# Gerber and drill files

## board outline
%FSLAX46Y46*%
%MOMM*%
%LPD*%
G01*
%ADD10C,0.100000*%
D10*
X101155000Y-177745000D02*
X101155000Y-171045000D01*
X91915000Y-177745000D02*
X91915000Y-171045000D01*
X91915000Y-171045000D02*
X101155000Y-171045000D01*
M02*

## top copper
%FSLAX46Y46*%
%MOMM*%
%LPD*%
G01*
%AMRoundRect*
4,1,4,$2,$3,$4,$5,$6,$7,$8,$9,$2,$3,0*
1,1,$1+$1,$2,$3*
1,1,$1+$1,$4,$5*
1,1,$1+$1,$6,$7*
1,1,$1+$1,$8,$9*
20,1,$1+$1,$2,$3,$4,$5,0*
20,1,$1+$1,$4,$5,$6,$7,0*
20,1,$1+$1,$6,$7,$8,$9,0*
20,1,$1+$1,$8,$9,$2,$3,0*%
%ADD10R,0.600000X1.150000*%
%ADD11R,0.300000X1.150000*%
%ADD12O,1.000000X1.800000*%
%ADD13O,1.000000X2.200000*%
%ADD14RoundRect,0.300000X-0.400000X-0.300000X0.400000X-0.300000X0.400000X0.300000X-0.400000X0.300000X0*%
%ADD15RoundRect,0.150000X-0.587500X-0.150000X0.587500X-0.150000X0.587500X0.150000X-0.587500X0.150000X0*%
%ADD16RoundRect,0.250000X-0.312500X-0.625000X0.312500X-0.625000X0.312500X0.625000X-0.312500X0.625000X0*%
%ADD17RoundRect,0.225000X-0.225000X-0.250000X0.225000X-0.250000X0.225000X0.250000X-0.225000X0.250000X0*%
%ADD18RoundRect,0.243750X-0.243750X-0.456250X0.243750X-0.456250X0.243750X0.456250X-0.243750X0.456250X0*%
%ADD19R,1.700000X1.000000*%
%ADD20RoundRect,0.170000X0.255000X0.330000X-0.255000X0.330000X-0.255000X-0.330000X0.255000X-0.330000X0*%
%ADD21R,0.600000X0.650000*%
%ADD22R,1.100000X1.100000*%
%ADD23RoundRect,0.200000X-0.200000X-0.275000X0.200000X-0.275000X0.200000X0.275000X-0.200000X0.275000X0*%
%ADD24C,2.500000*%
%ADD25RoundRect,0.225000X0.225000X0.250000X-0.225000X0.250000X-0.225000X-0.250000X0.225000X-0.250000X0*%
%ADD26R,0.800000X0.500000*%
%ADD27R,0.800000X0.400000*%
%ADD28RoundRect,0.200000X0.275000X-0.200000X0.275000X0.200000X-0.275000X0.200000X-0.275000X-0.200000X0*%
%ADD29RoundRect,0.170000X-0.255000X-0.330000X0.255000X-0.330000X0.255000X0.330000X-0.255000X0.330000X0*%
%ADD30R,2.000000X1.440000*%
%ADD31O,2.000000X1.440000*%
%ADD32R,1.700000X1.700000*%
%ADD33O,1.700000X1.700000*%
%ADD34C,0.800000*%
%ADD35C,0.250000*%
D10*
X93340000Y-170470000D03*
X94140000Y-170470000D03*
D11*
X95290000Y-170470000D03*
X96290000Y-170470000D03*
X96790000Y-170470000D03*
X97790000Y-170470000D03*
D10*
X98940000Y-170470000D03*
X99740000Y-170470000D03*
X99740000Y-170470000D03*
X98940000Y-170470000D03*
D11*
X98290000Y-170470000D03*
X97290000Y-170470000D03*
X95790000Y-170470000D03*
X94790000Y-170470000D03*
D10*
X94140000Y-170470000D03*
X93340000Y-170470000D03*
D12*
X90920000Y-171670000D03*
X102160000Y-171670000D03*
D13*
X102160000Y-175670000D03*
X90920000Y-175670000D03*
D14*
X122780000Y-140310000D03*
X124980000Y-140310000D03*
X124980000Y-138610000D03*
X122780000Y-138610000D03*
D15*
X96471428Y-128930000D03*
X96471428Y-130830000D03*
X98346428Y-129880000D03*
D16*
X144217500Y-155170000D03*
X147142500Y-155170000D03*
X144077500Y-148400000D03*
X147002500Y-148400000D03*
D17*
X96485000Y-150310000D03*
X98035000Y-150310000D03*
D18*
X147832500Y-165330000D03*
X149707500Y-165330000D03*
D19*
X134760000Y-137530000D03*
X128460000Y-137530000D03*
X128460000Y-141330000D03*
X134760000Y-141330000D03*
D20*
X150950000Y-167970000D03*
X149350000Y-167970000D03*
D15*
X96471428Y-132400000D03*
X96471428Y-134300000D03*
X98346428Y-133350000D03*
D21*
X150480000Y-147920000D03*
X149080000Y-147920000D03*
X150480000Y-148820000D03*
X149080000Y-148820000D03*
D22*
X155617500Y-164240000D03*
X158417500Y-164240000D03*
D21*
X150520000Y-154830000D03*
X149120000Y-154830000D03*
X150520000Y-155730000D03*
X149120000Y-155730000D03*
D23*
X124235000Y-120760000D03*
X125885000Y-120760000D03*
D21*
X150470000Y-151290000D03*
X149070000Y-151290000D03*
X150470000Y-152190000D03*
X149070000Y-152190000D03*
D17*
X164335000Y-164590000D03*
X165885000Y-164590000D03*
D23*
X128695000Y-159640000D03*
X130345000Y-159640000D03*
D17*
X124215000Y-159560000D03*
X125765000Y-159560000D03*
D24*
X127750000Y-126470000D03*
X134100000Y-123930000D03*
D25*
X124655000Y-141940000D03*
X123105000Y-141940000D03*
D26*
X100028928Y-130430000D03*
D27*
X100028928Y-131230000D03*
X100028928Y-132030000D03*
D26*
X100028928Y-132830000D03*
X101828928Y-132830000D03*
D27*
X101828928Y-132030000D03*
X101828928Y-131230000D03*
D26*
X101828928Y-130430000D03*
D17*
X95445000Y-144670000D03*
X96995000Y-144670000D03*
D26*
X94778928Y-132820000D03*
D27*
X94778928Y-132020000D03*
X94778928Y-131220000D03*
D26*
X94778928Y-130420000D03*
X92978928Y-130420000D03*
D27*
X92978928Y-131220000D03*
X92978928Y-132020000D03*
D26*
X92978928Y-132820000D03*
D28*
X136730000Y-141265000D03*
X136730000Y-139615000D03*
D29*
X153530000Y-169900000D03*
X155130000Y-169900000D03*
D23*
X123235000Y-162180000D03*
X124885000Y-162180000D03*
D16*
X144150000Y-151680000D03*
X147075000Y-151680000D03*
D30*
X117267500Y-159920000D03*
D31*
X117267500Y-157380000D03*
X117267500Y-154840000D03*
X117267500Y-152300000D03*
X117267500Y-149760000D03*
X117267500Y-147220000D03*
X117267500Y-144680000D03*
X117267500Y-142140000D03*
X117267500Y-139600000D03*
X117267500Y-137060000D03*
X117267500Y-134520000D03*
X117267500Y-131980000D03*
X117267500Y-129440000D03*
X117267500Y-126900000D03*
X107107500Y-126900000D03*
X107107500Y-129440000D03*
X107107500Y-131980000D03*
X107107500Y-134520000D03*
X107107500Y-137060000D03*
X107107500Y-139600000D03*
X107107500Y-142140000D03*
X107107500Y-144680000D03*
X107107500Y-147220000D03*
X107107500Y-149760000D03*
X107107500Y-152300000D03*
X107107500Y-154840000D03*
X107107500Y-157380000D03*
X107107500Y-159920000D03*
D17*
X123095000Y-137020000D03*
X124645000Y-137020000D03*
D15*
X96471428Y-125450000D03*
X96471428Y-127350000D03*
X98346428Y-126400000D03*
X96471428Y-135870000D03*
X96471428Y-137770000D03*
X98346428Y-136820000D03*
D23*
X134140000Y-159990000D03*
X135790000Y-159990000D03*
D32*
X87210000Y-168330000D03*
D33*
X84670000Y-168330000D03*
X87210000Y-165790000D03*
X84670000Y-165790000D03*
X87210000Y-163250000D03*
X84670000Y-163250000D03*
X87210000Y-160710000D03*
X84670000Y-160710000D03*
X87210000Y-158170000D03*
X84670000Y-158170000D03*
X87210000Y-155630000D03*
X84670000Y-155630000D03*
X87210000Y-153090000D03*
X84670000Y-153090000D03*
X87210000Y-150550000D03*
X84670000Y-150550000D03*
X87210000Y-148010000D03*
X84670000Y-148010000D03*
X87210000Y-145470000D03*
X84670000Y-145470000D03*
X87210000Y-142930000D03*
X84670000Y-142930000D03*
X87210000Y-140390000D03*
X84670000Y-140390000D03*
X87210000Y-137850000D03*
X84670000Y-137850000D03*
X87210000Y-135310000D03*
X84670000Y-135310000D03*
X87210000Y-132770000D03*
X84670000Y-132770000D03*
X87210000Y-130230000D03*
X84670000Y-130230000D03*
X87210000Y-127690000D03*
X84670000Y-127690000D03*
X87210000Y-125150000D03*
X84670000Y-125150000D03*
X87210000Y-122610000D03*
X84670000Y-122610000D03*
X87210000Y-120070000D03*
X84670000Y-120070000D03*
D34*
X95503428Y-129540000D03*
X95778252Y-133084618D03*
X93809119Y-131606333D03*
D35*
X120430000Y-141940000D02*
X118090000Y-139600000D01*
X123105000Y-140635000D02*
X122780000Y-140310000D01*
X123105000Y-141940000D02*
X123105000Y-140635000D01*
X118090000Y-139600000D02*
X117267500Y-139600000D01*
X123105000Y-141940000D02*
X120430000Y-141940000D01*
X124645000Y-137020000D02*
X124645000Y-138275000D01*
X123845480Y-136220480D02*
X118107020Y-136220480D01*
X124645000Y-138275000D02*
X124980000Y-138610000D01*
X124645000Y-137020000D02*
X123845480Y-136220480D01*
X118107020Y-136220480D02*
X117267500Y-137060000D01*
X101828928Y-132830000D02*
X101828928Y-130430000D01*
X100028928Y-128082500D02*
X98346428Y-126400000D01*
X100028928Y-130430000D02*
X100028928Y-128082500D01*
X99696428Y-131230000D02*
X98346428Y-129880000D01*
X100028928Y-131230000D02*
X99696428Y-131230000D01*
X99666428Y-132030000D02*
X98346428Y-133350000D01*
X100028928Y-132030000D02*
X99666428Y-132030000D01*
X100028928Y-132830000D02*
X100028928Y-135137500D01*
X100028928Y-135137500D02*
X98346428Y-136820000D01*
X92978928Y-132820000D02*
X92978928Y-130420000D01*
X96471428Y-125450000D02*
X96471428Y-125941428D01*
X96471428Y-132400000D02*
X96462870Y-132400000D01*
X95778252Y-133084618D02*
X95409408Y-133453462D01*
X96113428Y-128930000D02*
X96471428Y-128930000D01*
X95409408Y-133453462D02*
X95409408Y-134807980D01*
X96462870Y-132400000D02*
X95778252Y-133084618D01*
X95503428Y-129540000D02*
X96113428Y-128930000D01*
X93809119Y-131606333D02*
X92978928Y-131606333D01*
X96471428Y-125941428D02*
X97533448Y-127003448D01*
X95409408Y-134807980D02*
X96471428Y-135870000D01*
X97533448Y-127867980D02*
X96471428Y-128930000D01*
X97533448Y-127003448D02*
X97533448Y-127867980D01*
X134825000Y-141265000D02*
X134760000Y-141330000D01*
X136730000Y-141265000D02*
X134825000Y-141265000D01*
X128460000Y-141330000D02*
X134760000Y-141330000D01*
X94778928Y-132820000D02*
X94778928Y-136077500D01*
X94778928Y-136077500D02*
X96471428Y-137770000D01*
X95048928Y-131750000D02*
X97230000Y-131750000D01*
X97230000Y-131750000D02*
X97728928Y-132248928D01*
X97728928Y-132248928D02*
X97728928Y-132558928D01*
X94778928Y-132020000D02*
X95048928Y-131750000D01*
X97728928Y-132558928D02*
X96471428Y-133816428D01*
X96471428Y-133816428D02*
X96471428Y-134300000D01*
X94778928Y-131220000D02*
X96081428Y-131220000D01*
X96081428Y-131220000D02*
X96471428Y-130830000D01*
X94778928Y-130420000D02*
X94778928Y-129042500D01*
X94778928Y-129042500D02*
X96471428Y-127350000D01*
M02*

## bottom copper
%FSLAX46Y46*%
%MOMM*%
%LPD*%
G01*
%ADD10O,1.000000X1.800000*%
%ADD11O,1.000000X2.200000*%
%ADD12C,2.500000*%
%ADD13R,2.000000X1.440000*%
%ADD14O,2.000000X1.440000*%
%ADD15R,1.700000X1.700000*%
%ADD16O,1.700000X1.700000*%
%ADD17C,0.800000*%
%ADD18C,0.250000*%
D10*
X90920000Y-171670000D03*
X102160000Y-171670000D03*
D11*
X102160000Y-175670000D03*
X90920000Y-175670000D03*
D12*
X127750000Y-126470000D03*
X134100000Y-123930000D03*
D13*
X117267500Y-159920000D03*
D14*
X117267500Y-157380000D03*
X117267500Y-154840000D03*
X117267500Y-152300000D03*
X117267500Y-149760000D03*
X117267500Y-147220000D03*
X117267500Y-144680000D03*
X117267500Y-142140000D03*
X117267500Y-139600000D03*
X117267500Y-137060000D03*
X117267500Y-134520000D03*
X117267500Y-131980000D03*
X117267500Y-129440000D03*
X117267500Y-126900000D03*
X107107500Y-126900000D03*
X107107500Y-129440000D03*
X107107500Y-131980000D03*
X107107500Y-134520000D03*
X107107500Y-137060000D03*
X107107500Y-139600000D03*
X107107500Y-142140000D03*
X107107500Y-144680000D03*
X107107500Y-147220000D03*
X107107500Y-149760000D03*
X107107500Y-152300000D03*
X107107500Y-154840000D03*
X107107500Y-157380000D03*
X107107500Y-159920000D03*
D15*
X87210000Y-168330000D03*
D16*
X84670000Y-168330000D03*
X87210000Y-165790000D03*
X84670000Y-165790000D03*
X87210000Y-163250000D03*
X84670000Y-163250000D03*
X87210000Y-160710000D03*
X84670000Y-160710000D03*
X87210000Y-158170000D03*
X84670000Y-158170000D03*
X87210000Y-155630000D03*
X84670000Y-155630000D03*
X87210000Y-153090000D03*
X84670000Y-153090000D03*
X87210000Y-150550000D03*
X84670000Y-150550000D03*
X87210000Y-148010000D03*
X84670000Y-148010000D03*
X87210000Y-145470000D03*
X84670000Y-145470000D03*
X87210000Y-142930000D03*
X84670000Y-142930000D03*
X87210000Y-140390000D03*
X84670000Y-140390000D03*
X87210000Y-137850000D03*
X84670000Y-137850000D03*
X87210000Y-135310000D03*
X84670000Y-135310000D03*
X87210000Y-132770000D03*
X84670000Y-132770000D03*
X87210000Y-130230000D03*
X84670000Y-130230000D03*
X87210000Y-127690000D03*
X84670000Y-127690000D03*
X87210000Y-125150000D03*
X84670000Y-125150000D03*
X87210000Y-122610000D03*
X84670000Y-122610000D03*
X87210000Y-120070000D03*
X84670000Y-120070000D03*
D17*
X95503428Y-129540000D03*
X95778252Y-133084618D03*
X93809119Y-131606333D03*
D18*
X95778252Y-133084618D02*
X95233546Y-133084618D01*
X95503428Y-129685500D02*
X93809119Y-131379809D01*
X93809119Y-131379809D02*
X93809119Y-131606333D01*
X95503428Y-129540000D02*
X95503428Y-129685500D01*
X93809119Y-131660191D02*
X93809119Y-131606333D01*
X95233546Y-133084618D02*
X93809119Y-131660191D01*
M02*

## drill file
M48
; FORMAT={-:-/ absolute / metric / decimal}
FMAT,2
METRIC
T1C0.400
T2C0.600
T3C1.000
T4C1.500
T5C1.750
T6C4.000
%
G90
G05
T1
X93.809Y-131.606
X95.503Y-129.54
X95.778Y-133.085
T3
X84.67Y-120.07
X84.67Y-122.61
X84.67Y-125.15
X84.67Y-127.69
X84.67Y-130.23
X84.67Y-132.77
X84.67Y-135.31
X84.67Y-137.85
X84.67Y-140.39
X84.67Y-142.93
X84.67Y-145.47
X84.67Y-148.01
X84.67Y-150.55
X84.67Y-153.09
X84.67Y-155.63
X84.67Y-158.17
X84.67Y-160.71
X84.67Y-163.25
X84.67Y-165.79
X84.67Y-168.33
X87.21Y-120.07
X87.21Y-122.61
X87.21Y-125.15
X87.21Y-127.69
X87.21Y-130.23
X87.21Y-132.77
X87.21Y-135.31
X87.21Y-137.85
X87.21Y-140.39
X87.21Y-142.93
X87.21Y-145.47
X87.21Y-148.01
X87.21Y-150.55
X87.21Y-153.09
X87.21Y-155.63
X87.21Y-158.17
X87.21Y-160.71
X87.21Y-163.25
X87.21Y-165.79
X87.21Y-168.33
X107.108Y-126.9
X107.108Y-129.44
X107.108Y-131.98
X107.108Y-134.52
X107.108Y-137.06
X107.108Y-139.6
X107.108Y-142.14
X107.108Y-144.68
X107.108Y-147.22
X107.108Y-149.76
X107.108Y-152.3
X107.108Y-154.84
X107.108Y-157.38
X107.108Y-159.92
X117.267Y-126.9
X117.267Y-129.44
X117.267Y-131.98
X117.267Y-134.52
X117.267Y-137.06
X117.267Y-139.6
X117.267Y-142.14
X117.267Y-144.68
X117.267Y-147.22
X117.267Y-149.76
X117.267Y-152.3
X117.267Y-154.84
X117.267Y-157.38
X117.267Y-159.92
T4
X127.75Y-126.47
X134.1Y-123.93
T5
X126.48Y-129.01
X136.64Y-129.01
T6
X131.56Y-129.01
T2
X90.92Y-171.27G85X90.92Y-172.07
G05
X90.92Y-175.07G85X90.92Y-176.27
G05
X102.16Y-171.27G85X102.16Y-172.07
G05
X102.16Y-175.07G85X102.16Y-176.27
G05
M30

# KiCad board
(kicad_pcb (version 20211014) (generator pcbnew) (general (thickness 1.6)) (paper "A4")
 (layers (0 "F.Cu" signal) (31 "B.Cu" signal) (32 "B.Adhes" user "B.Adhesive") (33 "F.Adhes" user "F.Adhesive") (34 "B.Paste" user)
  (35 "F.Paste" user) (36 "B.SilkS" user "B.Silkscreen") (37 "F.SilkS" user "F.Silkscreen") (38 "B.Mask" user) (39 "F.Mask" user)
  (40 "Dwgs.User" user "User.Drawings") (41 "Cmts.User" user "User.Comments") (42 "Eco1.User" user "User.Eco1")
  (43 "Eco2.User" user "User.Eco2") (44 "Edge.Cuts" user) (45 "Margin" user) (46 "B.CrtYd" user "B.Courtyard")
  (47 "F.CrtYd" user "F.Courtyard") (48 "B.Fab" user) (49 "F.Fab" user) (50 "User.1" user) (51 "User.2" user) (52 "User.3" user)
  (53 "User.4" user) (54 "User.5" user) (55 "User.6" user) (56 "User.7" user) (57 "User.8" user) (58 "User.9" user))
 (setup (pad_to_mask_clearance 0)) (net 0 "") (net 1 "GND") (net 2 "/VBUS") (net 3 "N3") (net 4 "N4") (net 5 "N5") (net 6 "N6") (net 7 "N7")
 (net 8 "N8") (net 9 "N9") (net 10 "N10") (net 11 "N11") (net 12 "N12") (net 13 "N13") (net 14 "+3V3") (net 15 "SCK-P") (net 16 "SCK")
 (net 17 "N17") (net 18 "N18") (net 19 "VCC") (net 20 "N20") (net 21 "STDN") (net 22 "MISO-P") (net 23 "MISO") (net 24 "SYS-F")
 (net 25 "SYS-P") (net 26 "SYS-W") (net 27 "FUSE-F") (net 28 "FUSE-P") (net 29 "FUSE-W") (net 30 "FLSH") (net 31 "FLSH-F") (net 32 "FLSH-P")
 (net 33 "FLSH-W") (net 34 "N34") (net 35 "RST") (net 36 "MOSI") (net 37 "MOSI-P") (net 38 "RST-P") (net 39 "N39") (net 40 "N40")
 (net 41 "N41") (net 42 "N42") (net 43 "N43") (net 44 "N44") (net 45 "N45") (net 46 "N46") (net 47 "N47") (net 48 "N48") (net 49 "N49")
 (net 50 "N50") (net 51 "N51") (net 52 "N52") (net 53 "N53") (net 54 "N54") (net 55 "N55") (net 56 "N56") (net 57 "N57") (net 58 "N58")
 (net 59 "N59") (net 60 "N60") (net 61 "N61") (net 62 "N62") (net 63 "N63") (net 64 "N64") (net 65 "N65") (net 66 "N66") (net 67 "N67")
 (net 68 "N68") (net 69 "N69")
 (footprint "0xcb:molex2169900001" (layer "F.Cu") (at 96.54 177.77)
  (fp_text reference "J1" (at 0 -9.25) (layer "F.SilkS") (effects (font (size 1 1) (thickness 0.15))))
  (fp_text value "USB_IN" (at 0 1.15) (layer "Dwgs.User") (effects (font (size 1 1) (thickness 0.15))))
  (fp_line (start 4.615 -0.025) (end 4.615 -6.725) (layer "Edge.Cuts") (width 0.1))
  (fp_line (start -4.625 -0.025) (end -4.625 -6.725) (layer "Edge.Cuts") (width 0.1))
  (fp_line (start -4.625 -6.725) (end 4.615 -6.725) (layer "Edge.Cuts") (width 0.1))
  (pad "A1" smd rect (at -3.2 -7.3) (size 0.6 1.15) (layers "F.Cu" "F.Paste" "F.Mask") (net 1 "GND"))
  (pad "A4" smd rect (at -2.4 -7.3) (size 0.6 1.15) (layers "F.Cu" "F.Paste" "F.Mask") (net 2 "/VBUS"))
  (pad "A5" smd rect (at -1.25 -7.3) (size 0.3 1.15) (layers "F.Cu" "F.Paste" "F.Mask") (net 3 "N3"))
  (pad "A6" smd rect (at -0.25 -7.3) (size 0.3 1.15) (layers "F.Cu" "F.Paste" "F.Mask") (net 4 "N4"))
  (pad "A7" smd rect (at 0.25 -7.3) (size 0.3 1.15) (layers "F.Cu" "F.Paste" "F.Mask") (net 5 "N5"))
  (pad "A8" smd rect (at 1.25 -7.3) (size 0.3 1.15) (layers "F.Cu" "F.Paste" "F.Mask") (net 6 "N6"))
  (pad "A9" smd rect (at 2.4 -7.3) (size 0.6 1.15) (layers "F.Cu" "F.Paste" "F.Mask") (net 2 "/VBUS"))
  (pad "A12" smd rect (at 3.2 -7.3) (size 0.6 1.15) (layers "F.Cu" "F.Paste" "F.Mask") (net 1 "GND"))
  (pad "B1" smd rect (at 3.2 -7.3) (size 0.6 1.15) (layers "F.Cu" "F.Paste" "F.Mask") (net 1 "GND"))
  (pad "B4" smd rect (at 2.4 -7.3) (size 0.6 1.15) (layers "F.Cu" "F.Paste" "F.Mask") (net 2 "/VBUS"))
  (pad "B5" smd rect (at 1.75 -7.3) (size 0.3 1.15) (layers "F.Cu" "F.Paste" "F.Mask") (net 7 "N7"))
  (pad "B6" smd rect (at 0.75 -7.3) (size 0.3 1.15) (layers "F.Cu" "F.Paste" "F.Mask") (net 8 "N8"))
  (pad "B7" smd rect (at -0.75 -7.3) (size 0.3 1.15) (layers "F.Cu" "F.Paste" "F.Mask") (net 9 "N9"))
  (pad "B8" smd rect (at -1.75 -7.3) (size 0.3 1.15) (layers "F.Cu" "F.Paste" "F.Mask") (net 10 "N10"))
  (pad "B9" smd rect (at -2.4 -7.3) (size 0.6 1.15) (layers "F.Cu" "F.Paste" "F.Mask") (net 2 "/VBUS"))
  (pad "B12" smd rect (at -3.2 -7.3) (size 0.6 1.15) (layers "F.Cu" "F.Paste" "F.Mask") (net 1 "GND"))
  (pad "S1" thru_hole oval (at -5.62 -6.1) (size 1 1.8) (drill oval 0.6 1.4) (layers *.Cu *.Mask) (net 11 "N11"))
  (pad "S2" thru_hole oval (at 5.62 -6.1) (size 1 1.8) (drill oval 0.6 1.4) (layers *.Cu *.Mask))
  (pad "S3" thru_hole oval (at 5.62 -2.1) (size 1 2.2) (drill oval 0.6 1.8) (layers *.Cu *.Mask))
  (pad "S4" thru_hole oval (at -5.62 -2.1) (size 1 2.2) (drill oval 0.6 1.8) (layers *.Cu *.Mask)))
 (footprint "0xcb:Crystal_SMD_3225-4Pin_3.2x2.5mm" (layer "F.Cu") (at 123.88 139.46)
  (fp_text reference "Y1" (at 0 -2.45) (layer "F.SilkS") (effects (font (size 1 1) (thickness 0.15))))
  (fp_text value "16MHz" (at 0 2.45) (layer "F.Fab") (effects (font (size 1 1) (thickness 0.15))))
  (pad "1" smd roundrect (at -1.1 0.85) (size 1.4 1.2) (layers "F.Cu" "F.Paste" "F.Mask") (roundrect_rratio 0.25) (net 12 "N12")
   (solder_paste_margin_ratio -0.05))
  (pad "2" smd roundrect (at 1.1 0.85) (size 1.4 1.2) (layers "F.Cu" "F.Paste" "F.Mask") (roundrect_rratio 0.25) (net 1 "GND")
   (solder_paste_margin_ratio -0.05))
  (pad "3" smd roundrect (at 1.1 -0.85) (size 1.4 1.2) (layers "F.Cu" "F.Paste" "F.Mask") (roundrect_rratio 0.25) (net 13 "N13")
   (solder_paste_margin_ratio -0.05))
  (pad "4" smd roundrect (at -1.1 -0.85) (size 1.4 1.2) (layers "F.Cu" "F.Paste" "F.Mask") (roundrect_rratio 0.25) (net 1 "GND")
   (solder_paste_margin_ratio -0.05)))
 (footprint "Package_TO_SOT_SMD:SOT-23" (layer "F.Cu") (at 97.408928 129.88)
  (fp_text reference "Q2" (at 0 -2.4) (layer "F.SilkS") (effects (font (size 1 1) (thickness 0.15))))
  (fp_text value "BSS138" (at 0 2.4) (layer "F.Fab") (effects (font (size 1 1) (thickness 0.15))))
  (pad "1" smd roundrect locked (at -0.9375 -0.95) (size 1.475 0.6) (layers "F.Cu" "F.Paste" "F.Mask") (roundrect_rratio 0.25)
   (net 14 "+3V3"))
  (pad "2" smd roundrect locked (at -0.9375 0.95) (size 1.475 0.6) (layers "F.Cu" "F.Paste" "F.Mask") (roundrect_rratio 0.25)
   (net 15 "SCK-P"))
  (pad "3" smd roundrect locked (at 0.9375 0) (size 1.475 0.6) (layers "F.Cu" "F.Paste" "F.Mask") (roundrect_rratio 0.25) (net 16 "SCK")))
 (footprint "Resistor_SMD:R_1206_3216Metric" (layer "F.Cu") (at 145.68 155.17)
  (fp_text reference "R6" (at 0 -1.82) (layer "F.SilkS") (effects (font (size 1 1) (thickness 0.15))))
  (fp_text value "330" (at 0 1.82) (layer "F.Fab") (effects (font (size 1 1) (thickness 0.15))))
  (pad "1" smd roundrect locked (at -1.4625 0) (size 1.125 1.75) (layers "F.Cu" "F.Paste" "F.Mask") (roundrect_rratio 0.222222)
   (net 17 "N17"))
  (pad "2" smd roundrect locked (at 1.4625 0) (size 1.125 1.75) (layers "F.Cu" "F.Paste" "F.Mask") (roundrect_rratio 0.222222)
   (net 14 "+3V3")))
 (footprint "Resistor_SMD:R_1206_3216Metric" (layer "F.Cu") (at 145.54 148.4)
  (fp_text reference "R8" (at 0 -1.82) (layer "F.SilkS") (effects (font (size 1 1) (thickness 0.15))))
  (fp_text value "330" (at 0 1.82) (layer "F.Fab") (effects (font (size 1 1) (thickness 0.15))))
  (pad "1" smd roundrect locked (at -1.4625 0) (size 1.125 1.75) (layers "F.Cu" "F.Paste" "F.Mask") (roundrect_rratio 0.222222)
   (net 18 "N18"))
  (pad "2" smd roundrect locked (at 1.4625 0) (size 1.125 1.75) (layers "F.Cu" "F.Paste" "F.Mask") (roundrect_rratio 0.222222)
   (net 14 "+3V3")))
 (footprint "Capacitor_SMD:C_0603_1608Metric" (layer "F.Cu") (at 97.26 150.31)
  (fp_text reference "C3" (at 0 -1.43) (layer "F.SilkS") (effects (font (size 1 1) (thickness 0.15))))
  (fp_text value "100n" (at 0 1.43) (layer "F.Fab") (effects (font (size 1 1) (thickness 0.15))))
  (pad "1" smd roundrect locked (at -0.775 0) (size 0.9 0.95) (layers "F.Cu" "F.Paste" "F.Mask") (roundrect_rratio 0.25) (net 1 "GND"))
  (pad "2" smd roundrect locked (at 0.775 0) (size 0.9 0.95) (layers "F.Cu" "F.Paste" "F.Mask") (roundrect_rratio 0.25) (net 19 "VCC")))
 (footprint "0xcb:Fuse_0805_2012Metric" (layer "F.Cu") (at 148.77 165.33)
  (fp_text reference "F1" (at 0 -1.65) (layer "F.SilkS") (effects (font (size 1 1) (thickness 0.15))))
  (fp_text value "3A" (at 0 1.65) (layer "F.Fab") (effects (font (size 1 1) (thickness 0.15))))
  (pad "1" smd roundrect (at -0.9375 0) (size 0.975 1.4) (layers "F.Cu" "F.Paste" "F.Mask") (roundrect_rratio 0.25) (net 2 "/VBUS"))
  (pad "2" smd roundrect (at 0.9375 0) (size 0.975 1.4) (layers "F.Cu" "F.Paste" "F.Mask") (roundrect_rratio 0.25) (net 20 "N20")))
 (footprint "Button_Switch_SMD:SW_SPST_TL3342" (layer "F.Cu") (at 131.61 139.43)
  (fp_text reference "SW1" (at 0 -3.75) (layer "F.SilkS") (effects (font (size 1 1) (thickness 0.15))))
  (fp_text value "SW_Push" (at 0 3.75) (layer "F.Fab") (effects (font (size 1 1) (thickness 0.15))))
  (pad "1" smd rect locked (at 3.15 -1.9) (size 1.7 1) (layers "F.Cu" "F.Paste" "F.Mask") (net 1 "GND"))
  (pad "1" smd rect locked (at -3.15 -1.9) (size 1.7 1) (layers "F.Cu" "F.Paste" "F.Mask") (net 1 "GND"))
  (pad "2" smd rect locked (at -3.15 1.9) (size 1.7 1) (layers "F.Cu" "F.Paste" "F.Mask") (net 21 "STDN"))
  (pad "2" smd rect locked (at 3.15 1.9) (size 1.7 1) (layers "F.Cu" "F.Paste" "F.Mask") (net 21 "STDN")))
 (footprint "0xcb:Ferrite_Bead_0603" (layer "F.Cu") (at 150.15 167.97 180)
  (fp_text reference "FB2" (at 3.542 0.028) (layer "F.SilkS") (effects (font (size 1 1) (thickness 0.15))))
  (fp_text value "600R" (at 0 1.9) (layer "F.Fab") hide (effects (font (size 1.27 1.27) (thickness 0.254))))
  (pad "1" smd roundrect (at -0.8 0 180) (size 0.85 1) (layers "F.Cu" "F.Paste" "F.Mask") (roundrect_rratio 0.2) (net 20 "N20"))
  (pad "2" smd roundrect (at 0.8 0 180) (size 0.85 1) (layers "F.Cu" "F.Paste" "F.Mask") (roundrect_rratio 0.2) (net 19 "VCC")))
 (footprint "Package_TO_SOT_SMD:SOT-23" (layer "F.Cu") (at 97.408928 133.35)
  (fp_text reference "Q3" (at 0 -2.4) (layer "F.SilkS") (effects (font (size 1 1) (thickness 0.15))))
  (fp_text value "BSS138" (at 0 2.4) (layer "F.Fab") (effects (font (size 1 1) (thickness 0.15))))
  (pad "1" smd roundrect locked (at -0.9375 -0.95) (size 1.475 0.6) (layers "F.Cu" "F.Paste" "F.Mask") (roundrect_rratio 0.25)
   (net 14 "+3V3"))
  (pad "2" smd roundrect locked (at -0.9375 0.95) (size 1.475 0.6) (layers "F.Cu" "F.Paste" "F.Mask") (roundrect_rratio 0.25)
   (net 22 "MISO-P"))
  (pad "3" smd roundrect locked (at 0.9375 0) (size 1.475 0.6) (layers "F.Cu" "F.Paste" "F.Mask") (roundrect_rratio 0.25) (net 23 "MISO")))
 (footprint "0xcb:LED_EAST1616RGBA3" (layer "F.Cu") (at 149.78 148.37)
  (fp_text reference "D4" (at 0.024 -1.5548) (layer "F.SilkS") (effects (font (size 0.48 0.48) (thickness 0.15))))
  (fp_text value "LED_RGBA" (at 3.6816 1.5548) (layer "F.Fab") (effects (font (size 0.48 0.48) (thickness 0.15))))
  (pad "1" smd rect locked (at 0.7 -0.45) (size 0.6 0.65) (layers "F.Cu" "F.Paste" "F.Mask") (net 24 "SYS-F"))
  (pad "2" smd rect locked (at -0.7 -0.45) (size 0.6 0.65) (layers "F.Cu" "F.Paste" "F.Mask") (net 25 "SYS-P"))
  (pad "3" smd rect locked (at 0.7 0.45) (size 0.6 0.65) (layers "F.Cu" "F.Paste" "F.Mask") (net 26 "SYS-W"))
  (pad "4" smd rect locked (at -0.7 0.45) (size 0.6 0.65) (layers "F.Cu" "F.Paste" "F.Mask") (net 18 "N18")))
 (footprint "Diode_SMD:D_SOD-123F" (layer "F.Cu") (at 157.0175 164.24)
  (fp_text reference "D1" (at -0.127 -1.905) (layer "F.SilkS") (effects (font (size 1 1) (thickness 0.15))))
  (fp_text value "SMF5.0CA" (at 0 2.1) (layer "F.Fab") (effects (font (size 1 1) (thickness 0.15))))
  (pad "1" smd rect locked (at -1.4 0) (size 1.1 1.1) (layers "F.Cu" "F.Paste" "F.Mask") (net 1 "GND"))
  (pad "2" smd rect locked (at 1.4 0) (size 1.1 1.1) (layers "F.Cu" "F.Paste" "F.Mask") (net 20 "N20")))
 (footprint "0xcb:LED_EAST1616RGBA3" (layer "F.Cu") (at 149.82 155.28)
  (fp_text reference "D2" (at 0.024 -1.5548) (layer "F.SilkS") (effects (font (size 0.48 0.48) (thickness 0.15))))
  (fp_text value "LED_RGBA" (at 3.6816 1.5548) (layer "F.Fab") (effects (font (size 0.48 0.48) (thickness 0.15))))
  (pad "1" smd rect locked (at 0.7 -0.45) (size 0.6 0.65) (layers "F.Cu" "F.Paste" "F.Mask") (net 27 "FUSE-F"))
  (pad "2" smd rect locked (at -0.7 -0.45) (size 0.6 0.65) (layers "F.Cu" "F.Paste" "F.Mask") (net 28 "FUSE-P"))
  (pad "3" smd rect locked (at 0.7 0.45) (size 0.6 0.65) (layers "F.Cu" "F.Paste" "F.Mask") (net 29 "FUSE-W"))
  (pad "4" smd rect locked (at -0.7 0.45) (size 0.6 0.65) (layers "F.Cu" "F.Paste" "F.Mask") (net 17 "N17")))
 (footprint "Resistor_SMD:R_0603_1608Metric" (layer "F.Cu") (at 125.06 120.76)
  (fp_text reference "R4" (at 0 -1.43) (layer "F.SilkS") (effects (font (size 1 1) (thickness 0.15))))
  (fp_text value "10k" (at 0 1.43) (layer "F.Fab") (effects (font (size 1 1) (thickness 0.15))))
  (pad "1" smd roundrect locked (at -0.825 0) (size 0.8 0.95) (layers "F.Cu" "F.Paste" "F.Mask") (roundrect_rratio 0.25) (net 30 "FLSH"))
  (pad "2" smd roundrect locked (at 0.825 0) (size 0.8 0.95) (layers "F.Cu" "F.Paste" "F.Mask") (roundrect_rratio 0.25) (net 14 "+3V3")))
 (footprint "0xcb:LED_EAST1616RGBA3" (layer "F.Cu") (at 149.77 151.74)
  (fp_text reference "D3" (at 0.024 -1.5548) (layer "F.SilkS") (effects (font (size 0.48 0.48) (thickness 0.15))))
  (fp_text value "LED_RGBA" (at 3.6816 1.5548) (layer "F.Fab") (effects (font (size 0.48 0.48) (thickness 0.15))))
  (pad "1" smd rect locked (at 0.7 -0.45) (size 0.6 0.65) (layers "F.Cu" "F.Paste" "F.Mask") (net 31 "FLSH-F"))
  (pad "2" smd rect locked (at -0.7 -0.45) (size 0.6 0.65) (layers "F.Cu" "F.Paste" "F.Mask") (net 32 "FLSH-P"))
  (pad "3" smd rect locked (at 0.7 0.45) (size 0.6 0.65) (layers "F.Cu" "F.Paste" "F.Mask") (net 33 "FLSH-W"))
  (pad "4" smd rect locked (at -0.7 0.45) (size 0.6 0.65) (layers "F.Cu" "F.Paste" "F.Mask") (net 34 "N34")))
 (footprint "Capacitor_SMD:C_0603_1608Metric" (layer "F.Cu") (at 165.11 164.59)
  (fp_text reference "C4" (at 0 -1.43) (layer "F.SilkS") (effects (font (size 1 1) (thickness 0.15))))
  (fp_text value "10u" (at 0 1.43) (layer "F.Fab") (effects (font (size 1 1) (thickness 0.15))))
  (pad "1" smd roundrect locked (at -0.775 0) (size 0.9 0.95) (layers "F.Cu" "F.Paste" "F.Mask") (roundrect_rratio 0.25) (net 20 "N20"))
  (pad "2" smd roundrect locked (at 0.775 0) (size 0.9 0.95) (layers "F.Cu" "F.Paste" "F.Mask") (roundrect_rratio 0.25) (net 1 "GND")))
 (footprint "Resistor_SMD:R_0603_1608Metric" (layer "F.Cu") (at 129.52 159.64)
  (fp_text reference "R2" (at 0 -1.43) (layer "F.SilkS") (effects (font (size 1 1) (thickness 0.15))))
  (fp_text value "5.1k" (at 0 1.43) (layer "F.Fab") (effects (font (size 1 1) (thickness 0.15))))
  (pad "1" smd roundrect locked (at -0.825 0) (size 0.8 0.95) (layers "F.Cu" "F.Paste" "F.Mask") (roundrect_rratio 0.25) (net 1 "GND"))
  (pad "2" smd roundrect locked (at 0.825 0) (size 0.8 0.95) (layers "F.Cu" "F.Paste" "F.Mask") (roundrect_rratio 0.25) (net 7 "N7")))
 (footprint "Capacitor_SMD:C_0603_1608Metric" (layer "F.Cu") (at 124.99 159.56)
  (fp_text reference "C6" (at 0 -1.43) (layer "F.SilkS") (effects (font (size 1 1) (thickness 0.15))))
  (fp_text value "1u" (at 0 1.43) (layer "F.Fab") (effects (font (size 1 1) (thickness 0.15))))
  (pad "1" smd roundrect locked (at -0.775 0) (size 0.9 0.95) (layers "F.Cu" "F.Paste" "F.Mask") (roundrect_rratio 0.25) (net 19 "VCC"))
  (pad "2" smd roundrect locked (at 0.775 0) (size 0.9 0.95) (layers "F.Cu" "F.Paste" "F.Mask") (roundrect_rratio 0.25) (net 1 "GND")))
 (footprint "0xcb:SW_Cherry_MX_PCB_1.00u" (layer "F.Cu") (at 131.56 129.01)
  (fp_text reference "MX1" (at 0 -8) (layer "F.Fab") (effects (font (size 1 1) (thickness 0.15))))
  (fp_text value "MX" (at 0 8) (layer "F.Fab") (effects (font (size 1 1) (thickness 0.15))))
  (pad "" np_thru_hole circle (at -5.08 0) (size 1.75 1.75) (drill 1.75) (layers *.Cu *.Mask))
  (pad "" np_thru_hole circle (at 5.08 0) (size 1.75 1.75) (drill 1.75) (layers *.Cu *.Mask))
  (pad "" np_thru_hole circle (at 0 0) (size 4 4) (drill 4) (layers *.Cu *.Mask))
  (pad "1" thru_hole circle (at -3.81 -2.54) (size 2.5 2.5) (drill 1.5) (layers *.Cu *.Mask) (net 30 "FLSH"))
  (pad "2" thru_hole circle (at 2.54 -5.08) (size 2.5 2.5) (drill 1.5) (layers *.Cu *.Mask) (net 1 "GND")))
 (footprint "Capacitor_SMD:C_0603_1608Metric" (layer "F.Cu") (at 123.88 141.94 180)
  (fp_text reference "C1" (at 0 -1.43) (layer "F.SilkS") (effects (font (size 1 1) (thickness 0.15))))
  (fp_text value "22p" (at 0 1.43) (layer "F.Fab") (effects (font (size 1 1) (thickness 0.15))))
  (pad "1" smd roundrect locked (at -0.775 0 180) (size 0.9 0.95) (layers "F.Cu" "F.Paste" "F.Mask") (roundrect_rratio 0.25) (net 1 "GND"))
  (pad "2" smd roundrect locked (at 0.775 0 180) (size 0.9 0.95) (layers "F.Cu" "F.Paste" "F.Mask") (roundrect_rratio 0.25) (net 12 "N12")))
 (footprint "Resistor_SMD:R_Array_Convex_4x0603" (layer "F.Cu") (at 100.928928 131.63)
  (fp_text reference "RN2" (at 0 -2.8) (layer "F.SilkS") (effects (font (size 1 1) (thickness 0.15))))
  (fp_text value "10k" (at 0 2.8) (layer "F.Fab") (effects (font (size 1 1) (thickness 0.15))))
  (pad "1" smd rect locked (at -0.9 -1.2) (size 0.8 0.5) (layers "F.Cu" "F.Paste" "F.Mask") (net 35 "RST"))
  (pad "2" smd rect locked (at -0.9 -0.4) (size 0.8 0.4) (layers "F.Cu" "F.Paste" "F.Mask") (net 16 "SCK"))
  (pad "3" smd rect locked (at -0.9 0.4) (size 0.8 0.4) (layers "F.Cu" "F.Paste" "F.Mask") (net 23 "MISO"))
  (pad "4" smd rect locked (at -0.9 1.2) (size 0.8 0.5) (layers "F.Cu" "F.Paste" "F.Mask") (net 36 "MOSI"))
  (pad "5" smd rect locked (at 0.9 1.2) (size 0.8 0.5) (layers "F.Cu" "F.Paste" "F.Mask") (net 19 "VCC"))
  (pad "6" smd rect locked (at 0.9 0.4) (size 0.8 0.4) (layers "F.Cu" "F.Paste" "F.Mask") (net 19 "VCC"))
  (pad "7" smd rect locked (at 0.9 -0.4) (size 0.8 0.4) (layers "F.Cu" "F.Paste" "F.Mask") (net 19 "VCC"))
  (pad "8" smd rect locked (at 0.9 -1.2) (size 0.8 0.5) (layers "F.Cu" "F.Paste" "F.Mask") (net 19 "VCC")))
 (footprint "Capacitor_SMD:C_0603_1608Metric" (layer "F.Cu") (at 96.22 144.67)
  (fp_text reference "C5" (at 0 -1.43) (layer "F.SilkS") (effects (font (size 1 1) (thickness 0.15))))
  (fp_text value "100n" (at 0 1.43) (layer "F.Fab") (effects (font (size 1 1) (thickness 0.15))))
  (pad "1" smd roundrect locked (at -0.775 0) (size 0.9 0.95) (layers "F.Cu" "F.Paste" "F.Mask") (roundrect_rratio 0.25) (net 19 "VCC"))
  (pad "2" smd roundrect locked (at 0.775 0) (size 0.9 0.95) (layers "F.Cu" "F.Paste" "F.Mask") (roundrect_rratio 0.25) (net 1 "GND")))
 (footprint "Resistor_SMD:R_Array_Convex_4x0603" (layer "F.Cu") (at 93.878928 131.62 180)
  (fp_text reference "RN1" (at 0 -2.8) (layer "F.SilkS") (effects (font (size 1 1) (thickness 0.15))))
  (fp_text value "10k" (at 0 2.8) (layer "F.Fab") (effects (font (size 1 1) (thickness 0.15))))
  (pad "1" smd rect locked (at -0.9 -1.2 180) (size 0.8 0.5) (layers "F.Cu" "F.Paste" "F.Mask") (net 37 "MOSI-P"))
  (pad "2" smd rect locked (at -0.9 -0.4 180) (size 0.8 0.4) (layers "F.Cu" "F.Paste" "F.Mask") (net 22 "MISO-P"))
  (pad "3" smd rect locked (at -0.9 0.4 180) (size 0.8 0.4) (layers "F.Cu" "F.Paste" "F.Mask") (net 15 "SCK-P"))
  (pad "4" smd rect locked (at -0.9 1.2 180) (size 0.8 0.5) (layers "F.Cu" "F.Paste" "F.Mask") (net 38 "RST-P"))
  (pad "5" smd rect locked (at 0.9 1.2 180) (size 0.8 0.5) (layers "F.Cu" "F.Paste" "F.Mask") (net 14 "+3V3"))
  (pad "6" smd rect locked (at 0.9 0.4 180) (size 0.8 0.4) (layers "F.Cu" "F.Paste" "F.Mask") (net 14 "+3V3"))
  (pad "7" smd rect locked (at 0.9 -0.4 180) (size 0.8 0.4) (layers "F.Cu" "F.Paste" "F.Mask") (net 14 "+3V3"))
  (pad "8" smd rect locked (at 0.9 -1.2 180) (size 0.8 0.5) (layers "F.Cu" "F.Paste" "F.Mask") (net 14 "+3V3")))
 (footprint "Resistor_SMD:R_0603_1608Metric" (layer "F.Cu") (at 136.73 140.44 90)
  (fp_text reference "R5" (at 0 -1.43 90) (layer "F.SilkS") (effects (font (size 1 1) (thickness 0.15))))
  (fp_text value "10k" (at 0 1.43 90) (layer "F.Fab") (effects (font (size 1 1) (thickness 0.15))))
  (pad "1" smd roundrect locked (at -0.825 0 90) (size 0.8 0.95) (layers "F.Cu" "F.Paste" "F.Mask") (roundrect_rratio 0.25) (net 21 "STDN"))
  (pad "2" smd roundrect locked (at 0.825 0 90) (size 0.8 0.95) (layers "F.Cu" "F.Paste" "F.Mask") (roundrect_rratio 0.25) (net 14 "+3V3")))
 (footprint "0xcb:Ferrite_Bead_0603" (layer "F.Cu") (at 154.33 169.9)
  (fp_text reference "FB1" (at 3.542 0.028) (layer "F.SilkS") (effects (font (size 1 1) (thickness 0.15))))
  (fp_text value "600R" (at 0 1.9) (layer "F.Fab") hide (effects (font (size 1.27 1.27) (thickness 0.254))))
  (pad "1" smd roundrect (at -0.8 0) (size 0.85 1) (layers "F.Cu" "F.Paste" "F.Mask") (roundrect_rratio 0.2) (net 1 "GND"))
  (pad "2" smd roundrect (at 0.8 0) (size 0.85 1) (layers "F.Cu" "F.Paste" "F.Mask") (roundrect_rratio 0.2) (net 11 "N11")))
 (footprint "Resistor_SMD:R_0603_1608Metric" (layer "F.Cu") (at 124.06 162.18)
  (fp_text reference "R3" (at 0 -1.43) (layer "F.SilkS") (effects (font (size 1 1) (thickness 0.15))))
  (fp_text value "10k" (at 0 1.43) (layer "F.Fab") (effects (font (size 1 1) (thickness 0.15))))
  (pad "1" smd roundrect locked (at -0.825 0) (size 0.8 0.95) (layers "F.Cu" "F.Paste" "F.Mask") (roundrect_rratio 0.25) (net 19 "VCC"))
  (pad "2" smd roundrect locked (at 0.825 0) (size 0.8 0.95) (layers "F.Cu" "F.Paste" "F.Mask") (roundrect_rratio 0.25) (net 35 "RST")))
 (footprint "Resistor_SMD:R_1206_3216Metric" (layer "F.Cu") (at 145.6125 151.68)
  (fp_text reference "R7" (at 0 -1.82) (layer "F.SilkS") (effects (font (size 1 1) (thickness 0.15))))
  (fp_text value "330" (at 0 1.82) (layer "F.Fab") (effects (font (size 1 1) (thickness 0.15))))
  (pad "1" smd roundrect locked (at -1.4625 0) (size 1.125 1.75) (layers "F.Cu" "F.Paste" "F.Mask") (roundrect_rratio 0.222222)
   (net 34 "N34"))
  (pad "2" smd roundrect locked (at 1.4625 0) (size 1.125 1.75) (layers "F.Cu" "F.Paste" "F.Mask") (roundrect_rratio 0.222222)
   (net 14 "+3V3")))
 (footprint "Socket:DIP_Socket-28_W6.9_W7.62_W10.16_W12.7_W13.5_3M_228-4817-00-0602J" (layer "F.Cu") (at 117.2675 159.92 180)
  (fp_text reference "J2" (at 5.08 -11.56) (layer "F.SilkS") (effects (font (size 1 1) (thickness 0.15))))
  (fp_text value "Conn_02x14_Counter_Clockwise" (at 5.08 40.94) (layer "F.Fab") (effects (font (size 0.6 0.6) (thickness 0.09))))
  (pad "1" thru_hole rect locked (at 0 0 180) (size 2 1.44) (drill 1) (layers *.Cu *.Mask) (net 35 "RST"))
  (pad "2" thru_hole oval locked (at 0 2.54 180) (size 2 1.44) (drill 1) (layers *.Cu *.Mask) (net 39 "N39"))
  (pad "3" thru_hole oval locked (at 0 5.08 180) (size 2 1.44) (drill 1) (layers *.Cu *.Mask) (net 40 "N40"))
  (pad "4" thru_hole oval locked (at 0 7.62 180) (size 2 1.44) (drill 1) (layers *.Cu *.Mask) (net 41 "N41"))
  (pad "5" thru_hole oval locked (at 0 10.16 180) (size 2 1.44) (drill 1) (layers *.Cu *.Mask) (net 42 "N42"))
  (pad "6" thru_hole oval locked (at 0 12.7 180) (size 2 1.44) (drill 1) (layers *.Cu *.Mask) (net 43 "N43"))
  (pad "7" thru_hole oval locked (at 0 15.24 180) (size 2 1.44) (drill 1) (layers *.Cu *.Mask) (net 19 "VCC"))
  (pad "8" thru_hole oval locked (at 0 17.78 180) (size 2 1.44) (drill 1) (layers *.Cu *.Mask) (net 1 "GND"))
  (pad "9" thru_hole oval locked (at 0 20.32 180) (size 2 1.44) (drill 1) (layers *.Cu *.Mask) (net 12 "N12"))
  (pad "10" thru_hole oval locked (at 0 22.86 180) (size 2 1.44) (drill 1) (layers *.Cu *.Mask) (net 13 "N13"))
  (pad "11" thru_hole oval locked (at 0 25.4 180) (size 2 1.44) (drill 1) (layers *.Cu *.Mask) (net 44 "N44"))
  (pad "12" thru_hole oval locked (at 0 27.94 180) (size 2 1.44) (drill 1) (layers *.Cu *.Mask) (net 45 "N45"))
  (pad "13" thru_hole oval locked (at 0 30.48 180) (size 2 1.44) (drill 1) (layers *.Cu *.Mask) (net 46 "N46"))
  (pad "14" thru_hole oval locked (at 0 33.02 180) (size 2 1.44) (drill 1) (layers *.Cu *.Mask) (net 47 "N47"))
  (pad "15" thru_hole oval locked (at 10.16 33.02 180) (size 2 1.44) (drill 1) (layers *.Cu *.Mask) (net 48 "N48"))
  (pad "16" thru_hole oval locked (at 10.16 30.48 180) (size 2 1.44) (drill 1) (layers *.Cu *.Mask) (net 36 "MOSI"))
  (pad "17" thru_hole oval locked (at 10.16 27.94 180) (size 2 1.44) (drill 1) (layers *.Cu *.Mask) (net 23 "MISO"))
  (pad "18" thru_hole oval locked (at 10.16 25.4 180) (size 2 1.44) (drill 1) (layers *.Cu *.Mask) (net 16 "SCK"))
  (pad "19" thru_hole oval locked (at 10.16 22.86 180) (size 2 1.44) (drill 1) (layers *.Cu *.Mask) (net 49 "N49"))
  (pad "20" thru_hole oval locked (at 10.16 20.32 180) (size 2 1.44) (drill 1) (layers *.Cu *.Mask) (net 19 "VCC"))
  (pad "21" thru_hole oval locked (at 10.16 17.78 180) (size 2 1.44) (drill 1) (layers *.Cu *.Mask) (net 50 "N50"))
  (pad "22" thru_hole oval locked (at 10.16 15.24 180) (size 2 1.44) (drill 1) (layers *.Cu *.Mask) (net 1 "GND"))
  (pad "23" thru_hole oval locked (at 10.16 12.7 180) (size 2 1.44) (drill 1) (layers *.Cu *.Mask) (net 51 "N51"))
  (pad "24" thru_hole oval locked (at 10.16 10.16 180) (size 2 1.44) (drill 1) (layers *.Cu *.Mask) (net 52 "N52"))
  (pad "25" thru_hole oval locked (at 10.16 7.62 180) (size 2 1.44) (drill 1) (layers *.Cu *.Mask) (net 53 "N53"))
  (pad "26" thru_hole oval locked (at 10.16 5.08 180) (size 2 1.44) (drill 1) (layers *.Cu *.Mask) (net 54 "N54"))
  (pad "27" thru_hole oval locked (at 10.16 2.54 180) (size 2 1.44) (drill 1) (layers *.Cu *.Mask) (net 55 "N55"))
  (pad "28" thru_hole oval locked (at 10.16 0 180) (size 2 1.44) (drill 1) (layers *.Cu *.Mask) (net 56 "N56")))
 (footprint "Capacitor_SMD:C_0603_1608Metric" (layer "F.Cu") (at 123.87 137.02)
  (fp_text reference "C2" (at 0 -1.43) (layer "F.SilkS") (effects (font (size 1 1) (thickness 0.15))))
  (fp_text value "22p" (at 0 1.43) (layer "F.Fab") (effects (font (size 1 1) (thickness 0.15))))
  (pad "1" smd roundrect locked (at -0.775 0) (size 0.9 0.95) (layers "F.Cu" "F.Paste" "F.Mask") (roundrect_rratio 0.25) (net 1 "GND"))
  (pad "2" smd roundrect locked (at 0.775 0) (size 0.9 0.95) (layers "F.Cu" "F.Paste" "F.Mask") (roundrect_rratio 0.25) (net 13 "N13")))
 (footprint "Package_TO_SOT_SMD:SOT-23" (layer "F.Cu") (at 97.408928 126.4)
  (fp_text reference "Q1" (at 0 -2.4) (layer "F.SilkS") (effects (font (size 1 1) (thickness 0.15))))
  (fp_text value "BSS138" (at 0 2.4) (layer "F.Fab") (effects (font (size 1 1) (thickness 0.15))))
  (pad "1" smd roundrect locked (at -0.9375 -0.95) (size 1.475 0.6) (layers "F.Cu" "F.Paste" "F.Mask") (roundrect_rratio 0.25)
   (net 14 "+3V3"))
  (pad "2" smd roundrect locked (at -0.9375 0.95) (size 1.475 0.6) (layers "F.Cu" "F.Paste" "F.Mask") (roundrect_rratio 0.25)
   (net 38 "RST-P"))
  (pad "3" smd roundrect locked (at 0.9375 0) (size 1.475 0.6) (layers "F.Cu" "F.Paste" "F.Mask") (roundrect_rratio 0.25) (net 35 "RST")))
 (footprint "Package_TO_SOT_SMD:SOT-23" (layer "F.Cu") (at 97.408928 136.82)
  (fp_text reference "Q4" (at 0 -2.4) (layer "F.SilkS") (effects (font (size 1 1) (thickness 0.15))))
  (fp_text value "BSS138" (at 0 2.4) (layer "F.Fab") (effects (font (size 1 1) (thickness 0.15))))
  (pad "1" smd roundrect locked (at -0.9375 -0.95) (size 1.475 0.6) (layers "F.Cu" "F.Paste" "F.Mask") (roundrect_rratio 0.25)
   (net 14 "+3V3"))
  (pad "2" smd roundrect locked (at -0.9375 0.95) (size 1.475 0.6) (layers "F.Cu" "F.Paste" "F.Mask") (roundrect_rratio 0.25)
   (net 37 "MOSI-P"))
  (pad "3" smd roundrect locked (at 0.9375 0) (size 1.475 0.6) (layers "F.Cu" "F.Paste" "F.Mask") (roundrect_rratio 0.25) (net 36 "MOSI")))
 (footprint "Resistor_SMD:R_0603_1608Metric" (layer "F.Cu") (at 134.965 159.99)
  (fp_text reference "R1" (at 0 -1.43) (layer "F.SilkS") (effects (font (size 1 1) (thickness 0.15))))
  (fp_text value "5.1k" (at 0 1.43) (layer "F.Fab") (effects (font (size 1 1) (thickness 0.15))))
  (pad "1" smd roundrect locked (at -0.825 0) (size 0.8 0.95) (layers "F.Cu" "F.Paste" "F.Mask") (roundrect_rratio 0.25) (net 3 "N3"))
  (pad "2" smd roundrect locked (at 0.825 0) (size 0.8 0.95) (layers "F.Cu" "F.Paste" "F.Mask") (roundrect_rratio 0.25) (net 1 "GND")))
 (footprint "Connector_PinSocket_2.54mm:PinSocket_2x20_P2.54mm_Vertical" (layer "B.Cu") (at 87.21 168.33)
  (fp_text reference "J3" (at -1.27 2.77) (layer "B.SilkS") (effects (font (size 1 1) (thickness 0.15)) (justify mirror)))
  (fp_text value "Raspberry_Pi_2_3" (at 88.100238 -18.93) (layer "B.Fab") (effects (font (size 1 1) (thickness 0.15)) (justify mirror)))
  (pad "1" thru_hole rect locked (at 0 0) (size 1.7 1.7) (drill 1) (layers *.Cu *.Mask) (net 14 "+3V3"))
  (pad "2" thru_hole oval locked (at -2.54 0) (size 1.7 1.7) (drill 1) (layers *.Cu *.Mask) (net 19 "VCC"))
  (pad "3" thru_hole oval locked (at 0 -2.54) (size 1.7 1.7) (drill 1) (layers *.Cu *.Mask) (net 21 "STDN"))
  (pad "4" thru_hole oval locked (at -2.54 -2.54) (size 1.7 1.7) (drill 1) (layers *.Cu *.Mask) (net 19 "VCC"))
  (pad "5" thru_hole oval locked (at 0 -5.08) (size 1.7 1.7) (drill 1) (layers *.Cu *.Mask) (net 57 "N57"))
  (pad "6" thru_hole oval locked (at -2.54 -5.08) (size 1.7 1.7) (drill 1) (layers *.Cu *.Mask) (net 1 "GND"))
  (pad "7" thru_hole oval locked (at 0 -7.62) (size 1.7 1.7) (drill 1) (layers *.Cu *.Mask) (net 30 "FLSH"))
  (pad "8" thru_hole oval locked (at -2.54 -7.62) (size 1.7 1.7) (drill 1) (layers *.Cu *.Mask) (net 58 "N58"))
  (pad "9" thru_hole oval locked (at 0 -10.16) (size 1.7 1.7) (drill 1) (layers *.Cu *.Mask) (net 1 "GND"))
  (pad "10" thru_hole oval locked (at -2.54 -10.16) (size 1.7 1.7) (drill 1) (layers *.Cu *.Mask) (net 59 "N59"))
  (pad "11" thru_hole oval locked (at 0 -12.7) (size 1.7 1.7) (drill 1) (layers *.Cu *.Mask) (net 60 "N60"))
  (pad "12" thru_hole oval locked (at -2.54 -12.7) (size 1.7 1.7) (drill 1) (layers *.Cu *.Mask) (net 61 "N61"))
  (pad "13" thru_hole oval locked (at 0 -15.24) (size 1.7 1.7) (drill 1) (layers *.Cu *.Mask) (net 26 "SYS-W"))
  (pad "14" thru_hole oval locked (at -2.54 -15.24) (size 1.7 1.7) (drill 1) (layers *.Cu *.Mask) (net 1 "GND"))
  (pad "15" thru_hole oval locked (at 0 -17.78) (size 1.7 1.7) (drill 1) (layers *.Cu *.Mask) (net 27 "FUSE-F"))
  (pad "16" thru_hole oval locked (at -2.54 -17.78) (size 1.7 1.7) (drill 1) (layers *.Cu *.Mask) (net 28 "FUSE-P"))
  (pad "17" thru_hole oval locked (at 0 -20.32) (size 1.7 1.7) (drill 1) (layers *.Cu *.Mask) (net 14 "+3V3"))
  (pad "18" thru_hole oval locked (at -2.54 -20.32) (size 1.7 1.7) (drill 1) (layers *.Cu *.Mask) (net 31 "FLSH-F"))
  (pad "19" thru_hole oval locked (at 0 -22.86) (size 1.7 1.7) (drill 1) (layers *.Cu *.Mask) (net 37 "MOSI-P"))
  (pad "20" thru_hole oval locked (at -2.54 -22.86) (size 1.7 1.7) (drill 1) (layers *.Cu *.Mask) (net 1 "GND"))
  (pad "21" thru_hole oval locked (at 0 -25.4) (size 1.7 1.7) (drill 1) (layers *.Cu *.Mask) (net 22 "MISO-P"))
  (pad "22" thru_hole oval locked (at -2.54 -25.4) (size 1.7 1.7) (drill 1) (layers *.Cu *.Mask) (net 32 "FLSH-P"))
  (pad "23" thru_hole oval locked (at 0 -27.94) (size 1.7 1.7) (drill 1) (layers *.Cu *.Mask) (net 15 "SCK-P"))
  (pad "24" thru_hole oval locked (at -2.54 -27.94) (size 1.7 1.7) (drill 1) (layers *.Cu *.Mask) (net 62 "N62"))
  (pad "25" thru_hole oval locked (at 0 -30.48) (size 1.7 1.7) (drill 1) (layers *.Cu *.Mask) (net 1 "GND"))
  (pad "26" thru_hole oval locked (at -2.54 -30.48) (size 1.7 1.7) (drill 1) (layers *.Cu *.Mask) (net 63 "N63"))
  (pad "27" thru_hole oval locked (at 0 -33.02) (size 1.7 1.7) (drill 1) (layers *.Cu *.Mask) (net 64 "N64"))
  (pad "28" thru_hole oval locked (at -2.54 -33.02) (size 1.7 1.7) (drill 1) (layers *.Cu *.Mask) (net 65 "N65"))
  (pad "29" thru_hole oval locked (at 0 -35.56) (size 1.7 1.7) (drill 1) (layers *.Cu *.Mask) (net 29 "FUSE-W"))
  (pad "30" thru_hole oval locked (at -2.54 -35.56) (size 1.7 1.7) (drill 1) (layers *.Cu *.Mask) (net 1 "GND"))
  (pad "31" thru_hole oval locked (at 0 -38.1) (size 1.7 1.7) (drill 1) (layers *.Cu *.Mask) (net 33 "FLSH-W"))
  (pad "32" thru_hole oval locked (at -2.54 -38.1) (size 1.7 1.7) (drill 1) (layers *.Cu *.Mask) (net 24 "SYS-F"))
  (pad "33" thru_hole oval locked (at 0 -40.64) (size 1.7 1.7) (drill 1) (layers *.Cu *.Mask) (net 25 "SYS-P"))
  (pad "34" thru_hole oval locked (at -2.54 -40.64) (size 1.7 1.7) (drill 1) (layers *.Cu *.Mask) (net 1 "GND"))
  (pad "35" thru_hole oval locked (at 0 -43.18) (size 1.7 1.7) (drill 1) (layers *.Cu *.Mask) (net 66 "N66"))
  (pad "36" thru_hole oval locked (at -2.54 -43.18) (size 1.7 1.7) (drill 1) (layers *.Cu *.Mask) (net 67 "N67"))
  (pad "37" thru_hole oval locked (at 0 -45.72) (size 1.7 1.7) (drill 1) (layers *.Cu *.Mask) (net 38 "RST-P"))
  (pad "38" thru_hole oval locked (at -2.54 -45.72) (size 1.7 1.7) (drill 1) (layers *.Cu *.Mask) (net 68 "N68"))
  (pad "39" thru_hole oval locked (at 0 -48.26) (size 1.7 1.7) (drill 1) (layers *.Cu *.Mask) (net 1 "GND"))
  (pad "40" thru_hole oval locked (at -2.54 -48.26) (size 1.7 1.7) (drill 1) (layers *.Cu *.Mask) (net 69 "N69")))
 (segment (start 120.43 141.94) (end 118.09 139.6) (width 0.25) (layer "F.Cu") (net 12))
 (segment (start 123.105 140.635) (end 122.78 140.31) (width 0.25) (layer "F.Cu") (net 12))
 (segment (start 123.105 141.94) (end 123.105 140.635) (width 0.25) (layer "F.Cu") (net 12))
 (segment (start 118.09 139.6) (end 117.2675 139.6) (width 0.25) (layer "F.Cu") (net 12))
 (segment (start 123.105 141.94) (end 120.43 141.94) (width 0.25) (layer "F.Cu") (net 12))
 (segment (start 124.645 137.02) (end 124.645 138.275) (width 0.25) (layer "F.Cu") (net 13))
 (segment (start 123.84548 136.22048) (end 118.10702 136.22048) (width 0.25) (layer "F.Cu") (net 13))
 (segment (start 124.645 138.275) (end 124.98 138.61) (width 0.25) (layer "F.Cu") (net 13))
 (segment (start 124.645 137.02) (end 123.84548 136.22048) (width 0.25) (layer "F.Cu") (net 13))
 (segment (start 118.10702 136.22048) (end 117.2675 137.06) (width 0.25) (layer "F.Cu") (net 13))
 (segment (start 101.828928 132.83) (end 101.828928 130.43) (width 0.25) (layer "F.Cu") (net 19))
 (segment (start 100.028928 128.0825) (end 98.346428 126.4) (width 0.25) (layer "F.Cu") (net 35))
 (segment (start 100.028928 130.43) (end 100.028928 128.0825) (width 0.25) (layer "F.Cu") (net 35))
 (segment (start 99.696428 131.23) (end 98.346428 129.88) (width 0.25) (layer "F.Cu") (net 16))
 (segment (start 100.028928 131.23) (end 99.696428 131.23) (width 0.25) (layer "F.Cu") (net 16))
 (segment (start 99.666428 132.03) (end 98.346428 133.35) (width 0.25) (layer "F.Cu") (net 23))
 (segment (start 100.028928 132.03) (end 99.666428 132.03) (width 0.25) (layer "F.Cu") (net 23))
 (segment (start 100.028928 132.83) (end 100.028928 135.1375) (width 0.25) (layer "F.Cu") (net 36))
 (segment (start 100.028928 135.1375) (end 98.346428 136.82) (width 0.25) (layer "F.Cu") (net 36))
 (segment (start 92.978928 132.82) (end 92.978928 130.42) (width 0.25) (layer "F.Cu") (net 14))
 (segment (start 96.471428 125.45) (end 96.471428 125.941428) (width 0.25) (layer "F.Cu") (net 14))
 (segment (start 96.471428 132.4) (end 96.46287 132.4) (width 0.25) (layer "F.Cu") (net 14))
 (segment (start 95.778252 133.084618) (end 95.409408 133.453462) (width 0.25) (layer "F.Cu") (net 14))
 (segment (start 96.113428 128.93) (end 96.471428 128.93) (width 0.25) (layer "F.Cu") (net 14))
 (segment (start 95.409408 133.453462) (end 95.409408 134.80798) (width 0.25) (layer "F.Cu") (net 14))
 (segment (start 96.46287 132.4) (end 95.778252 133.084618) (width 0.25) (layer "F.Cu") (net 14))
 (segment (start 95.503428 129.54) (end 96.113428 128.93) (width 0.25) (layer "F.Cu") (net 14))
 (segment (start 93.809119 131.606333) (end 92.978928 131.606333) (width 0.25) (layer "F.Cu") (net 14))
 (segment (start 96.471428 125.941428) (end 97.533448 127.003448) (width 0.25) (layer "F.Cu") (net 14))
 (segment (start 95.409408 134.80798) (end 96.471428 135.87) (width 0.25) (layer "F.Cu") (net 14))
 (segment (start 97.533448 127.86798) (end 96.471428 128.93) (width 0.25) (layer "F.Cu") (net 14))
 (segment (start 97.533448 127.003448) (end 97.533448 127.86798) (width 0.25) (layer "F.Cu") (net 14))
 (via (at 95.503428 129.54) (size 0.8) (drill 0.4) (layers "F.Cu" "B.Cu") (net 14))
 (via (at 95.778252 133.084618) (size 0.8) (drill 0.4) (layers "F.Cu" "B.Cu") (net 14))
 (via (at 93.809119 131.606333) (size 0.8) (drill 0.4) (layers "F.Cu" "B.Cu") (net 14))
 (segment (start 95.778252 133.084618) (end 95.233546 133.084618) (width 0.25) (layer "B.Cu") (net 14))
 (segment (start 95.503428 129.6855) (end 93.809119 131.379809) (width 0.25) (layer "B.Cu") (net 14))
 (segment (start 93.809119 131.379809) (end 93.809119 131.606333) (width 0.25) (layer "B.Cu") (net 14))
 (segment (start 95.503428 129.54) (end 95.503428 129.6855) (width 0.25) (layer "B.Cu") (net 14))
 (segment (start 93.809119 131.660191) (end 93.809119 131.606333) (width 0.25) (layer "B.Cu") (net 14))
 (segment (start 95.233546 133.084618) (end 93.809119 131.660191) (width 0.25) (layer "B.Cu") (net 14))
 (segment (start 134.825 141.265) (end 134.76 141.33) (width 0.25) (layer "F.Cu") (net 21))
 (segment (start 136.73 141.265) (end 134.825 141.265) (width 0.25) (layer "F.Cu") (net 21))
 (segment (start 128.46 141.33) (end 134.76 141.33) (width 0.25) (layer "F.Cu") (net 21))
 (segment (start 94.778928 132.82) (end 94.778928 136.0775) (width 0.25) (layer "F.Cu") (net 37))
 (segment (start 94.778928 136.0775) (end 96.471428 137.77) (width 0.25) (layer "F.Cu") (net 37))
 (segment (start 95.048928 131.75) (end 97.23 131.75) (width 0.25) (layer "F.Cu") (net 22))
 (segment (start 97.23 131.75) (end 97.728928 132.248928) (width 0.25) (layer "F.Cu") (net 22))
 (segment (start 97.728928 132.248928) (end 97.728928 132.558928) (width 0.25) (layer "F.Cu") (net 22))
 (segment (start 94.778928 132.02) (end 95.048928 131.75) (width 0.25) (layer "F.Cu") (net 22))
 (segment (start 97.728928 132.558928) (end 96.471428 133.816428) (width 0.25) (layer "F.Cu") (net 22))
 (segment (start 96.471428 133.816428) (end 96.471428 134.3) (width 0.25) (layer "F.Cu") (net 22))
 (segment (start 94.778928 131.22) (end 96.081428 131.22) (width 0.25) (layer "F.Cu") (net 15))
 (segment (start 96.081428 131.22) (end 96.471428 130.83) (width 0.25) (layer "F.Cu") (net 15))
 (segment (start 94.778928 130.42) (end 94.778928 129.0425) (width 0.25) (layer "F.Cu") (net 38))
 (segment (start 94.778928 129.0425) (end 96.471428 127.35) (width 0.25) (layer "F.Cu") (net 38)))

